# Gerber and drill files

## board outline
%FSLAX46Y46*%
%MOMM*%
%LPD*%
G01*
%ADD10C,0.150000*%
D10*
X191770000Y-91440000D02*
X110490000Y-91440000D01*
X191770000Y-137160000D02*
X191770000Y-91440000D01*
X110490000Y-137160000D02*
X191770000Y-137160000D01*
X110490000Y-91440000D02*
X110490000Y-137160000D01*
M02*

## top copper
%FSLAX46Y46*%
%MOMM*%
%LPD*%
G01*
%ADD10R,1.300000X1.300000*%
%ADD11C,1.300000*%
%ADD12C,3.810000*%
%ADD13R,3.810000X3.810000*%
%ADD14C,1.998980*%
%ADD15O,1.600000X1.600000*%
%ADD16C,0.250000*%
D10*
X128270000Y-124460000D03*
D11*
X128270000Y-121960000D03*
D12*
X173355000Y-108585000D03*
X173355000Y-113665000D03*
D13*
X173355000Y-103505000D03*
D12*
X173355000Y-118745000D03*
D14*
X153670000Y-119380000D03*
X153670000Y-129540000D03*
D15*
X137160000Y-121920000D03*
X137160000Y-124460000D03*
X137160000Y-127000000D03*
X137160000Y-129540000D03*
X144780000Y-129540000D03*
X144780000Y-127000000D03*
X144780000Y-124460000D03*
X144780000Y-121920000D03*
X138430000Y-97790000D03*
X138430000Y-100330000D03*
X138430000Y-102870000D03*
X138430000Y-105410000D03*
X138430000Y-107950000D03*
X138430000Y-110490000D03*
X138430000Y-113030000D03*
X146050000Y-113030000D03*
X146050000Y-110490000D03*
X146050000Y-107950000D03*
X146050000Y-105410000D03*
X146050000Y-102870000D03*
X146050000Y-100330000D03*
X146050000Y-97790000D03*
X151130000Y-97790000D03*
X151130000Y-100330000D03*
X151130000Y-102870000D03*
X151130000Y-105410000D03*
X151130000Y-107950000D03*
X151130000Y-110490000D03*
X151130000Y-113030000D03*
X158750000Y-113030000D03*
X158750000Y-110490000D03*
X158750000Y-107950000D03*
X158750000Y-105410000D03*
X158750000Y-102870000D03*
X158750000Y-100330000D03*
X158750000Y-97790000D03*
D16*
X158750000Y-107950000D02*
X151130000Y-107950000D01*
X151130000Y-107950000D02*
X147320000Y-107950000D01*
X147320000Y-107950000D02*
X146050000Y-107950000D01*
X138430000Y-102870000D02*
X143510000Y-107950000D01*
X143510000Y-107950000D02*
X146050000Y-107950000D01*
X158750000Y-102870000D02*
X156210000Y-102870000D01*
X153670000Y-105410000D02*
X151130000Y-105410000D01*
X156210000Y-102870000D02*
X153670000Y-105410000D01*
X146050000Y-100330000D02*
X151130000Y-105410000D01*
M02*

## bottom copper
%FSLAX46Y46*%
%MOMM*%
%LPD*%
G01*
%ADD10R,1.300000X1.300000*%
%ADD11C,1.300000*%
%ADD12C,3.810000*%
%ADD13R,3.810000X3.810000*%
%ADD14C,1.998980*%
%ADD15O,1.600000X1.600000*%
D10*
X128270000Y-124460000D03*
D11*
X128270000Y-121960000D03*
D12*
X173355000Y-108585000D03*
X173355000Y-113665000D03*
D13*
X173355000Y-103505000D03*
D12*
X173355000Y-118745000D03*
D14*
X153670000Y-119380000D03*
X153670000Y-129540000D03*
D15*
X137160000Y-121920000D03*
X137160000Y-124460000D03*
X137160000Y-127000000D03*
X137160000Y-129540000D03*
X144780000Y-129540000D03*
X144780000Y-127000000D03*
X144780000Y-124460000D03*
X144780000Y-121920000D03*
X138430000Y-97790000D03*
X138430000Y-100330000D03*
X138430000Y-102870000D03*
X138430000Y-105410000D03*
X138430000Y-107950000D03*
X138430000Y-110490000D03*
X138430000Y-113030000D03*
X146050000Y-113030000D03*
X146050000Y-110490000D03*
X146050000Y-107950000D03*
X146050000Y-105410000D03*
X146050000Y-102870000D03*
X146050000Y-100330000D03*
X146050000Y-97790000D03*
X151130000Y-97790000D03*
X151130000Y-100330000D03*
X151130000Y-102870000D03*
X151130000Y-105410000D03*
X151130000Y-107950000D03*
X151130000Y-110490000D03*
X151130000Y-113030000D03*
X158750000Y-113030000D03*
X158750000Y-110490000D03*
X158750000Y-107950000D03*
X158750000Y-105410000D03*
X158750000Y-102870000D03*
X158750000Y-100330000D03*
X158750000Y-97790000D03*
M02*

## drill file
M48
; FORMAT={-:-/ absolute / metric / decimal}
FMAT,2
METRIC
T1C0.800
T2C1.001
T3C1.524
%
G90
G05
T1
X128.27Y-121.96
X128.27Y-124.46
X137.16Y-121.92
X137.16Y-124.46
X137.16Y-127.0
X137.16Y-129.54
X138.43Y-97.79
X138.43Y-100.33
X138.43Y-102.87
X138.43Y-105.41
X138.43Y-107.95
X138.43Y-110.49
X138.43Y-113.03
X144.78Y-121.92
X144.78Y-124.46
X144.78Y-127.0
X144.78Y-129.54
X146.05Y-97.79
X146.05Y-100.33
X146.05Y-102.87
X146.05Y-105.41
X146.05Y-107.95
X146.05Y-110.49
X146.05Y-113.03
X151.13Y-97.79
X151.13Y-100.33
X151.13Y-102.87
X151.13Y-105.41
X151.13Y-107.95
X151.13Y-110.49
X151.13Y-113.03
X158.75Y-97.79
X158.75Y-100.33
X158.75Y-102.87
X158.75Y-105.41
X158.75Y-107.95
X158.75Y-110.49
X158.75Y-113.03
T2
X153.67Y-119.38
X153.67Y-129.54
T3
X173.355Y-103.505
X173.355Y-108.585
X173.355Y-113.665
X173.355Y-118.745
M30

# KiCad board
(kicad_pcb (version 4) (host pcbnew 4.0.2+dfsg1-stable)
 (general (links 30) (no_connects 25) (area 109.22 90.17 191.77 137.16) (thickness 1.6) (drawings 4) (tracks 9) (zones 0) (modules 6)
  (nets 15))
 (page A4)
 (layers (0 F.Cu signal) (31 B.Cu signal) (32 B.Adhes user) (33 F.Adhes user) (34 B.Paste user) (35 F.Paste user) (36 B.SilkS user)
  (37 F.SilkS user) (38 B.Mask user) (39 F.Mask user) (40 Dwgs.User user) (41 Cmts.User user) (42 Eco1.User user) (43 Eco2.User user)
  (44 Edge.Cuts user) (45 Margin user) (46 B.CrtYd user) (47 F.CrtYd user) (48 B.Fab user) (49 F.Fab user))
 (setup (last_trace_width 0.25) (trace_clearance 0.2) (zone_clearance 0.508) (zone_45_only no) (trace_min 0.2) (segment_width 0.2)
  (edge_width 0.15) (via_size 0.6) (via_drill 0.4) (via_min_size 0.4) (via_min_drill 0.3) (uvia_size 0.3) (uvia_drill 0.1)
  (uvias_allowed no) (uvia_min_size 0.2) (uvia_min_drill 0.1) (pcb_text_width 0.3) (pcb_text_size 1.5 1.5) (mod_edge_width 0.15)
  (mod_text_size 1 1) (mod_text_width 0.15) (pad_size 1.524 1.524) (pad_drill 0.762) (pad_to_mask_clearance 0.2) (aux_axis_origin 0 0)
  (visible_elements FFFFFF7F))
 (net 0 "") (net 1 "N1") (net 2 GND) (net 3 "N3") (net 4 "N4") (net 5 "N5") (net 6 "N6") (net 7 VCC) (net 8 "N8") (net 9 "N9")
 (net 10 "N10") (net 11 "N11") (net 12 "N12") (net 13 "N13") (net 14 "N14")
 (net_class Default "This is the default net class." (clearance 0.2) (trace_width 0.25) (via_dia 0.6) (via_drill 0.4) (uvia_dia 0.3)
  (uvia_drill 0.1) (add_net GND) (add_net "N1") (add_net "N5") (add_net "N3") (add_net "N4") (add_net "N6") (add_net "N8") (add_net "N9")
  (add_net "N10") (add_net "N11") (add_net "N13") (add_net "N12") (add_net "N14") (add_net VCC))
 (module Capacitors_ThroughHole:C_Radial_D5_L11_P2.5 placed (layer F.Cu) (at 128.27 124.46 90)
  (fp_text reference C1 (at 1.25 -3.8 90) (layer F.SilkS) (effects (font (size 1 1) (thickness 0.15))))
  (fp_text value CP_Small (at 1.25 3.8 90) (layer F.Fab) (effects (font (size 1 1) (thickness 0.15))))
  (pad 1 thru_hole rect (at 0 0 90) (size 1.3 1.3) (drill 0.8) (layers *.Cu *.Mask F.SilkS) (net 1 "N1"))
  (pad 2 thru_hole circle (at 2.5 0 90) (size 1.3 1.3) (drill 0.8) (layers *.Cu *.Mask F.SilkS) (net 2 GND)))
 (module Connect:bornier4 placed (layer F.Cu) (at 173.355 111.125 270)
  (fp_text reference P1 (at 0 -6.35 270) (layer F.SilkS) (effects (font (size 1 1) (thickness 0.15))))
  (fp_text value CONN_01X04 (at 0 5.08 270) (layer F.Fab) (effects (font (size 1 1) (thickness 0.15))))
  (pad 2 thru_hole circle (at -2.54 0 270) (size 3.81 3.81) (drill 1.524) (layers *.Cu *.Mask F.SilkS) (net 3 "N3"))
  (pad 3 thru_hole circle (at 2.54 0 270) (size 3.81 3.81) (drill 1.524) (layers *.Cu *.Mask F.SilkS) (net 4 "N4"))
  (pad 1 thru_hole rect (at -7.62 0 270) (size 3.81 3.81) (drill 1.524) (layers *.Cu *.Mask F.SilkS) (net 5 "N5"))
  (pad 4 thru_hole circle (at 7.62 0 270) (size 3.81 3.81) (drill 1.524) (layers *.Cu *.Mask F.SilkS) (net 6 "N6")))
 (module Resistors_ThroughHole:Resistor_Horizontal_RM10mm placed (layer F.Cu) (at 153.67 119.38 270)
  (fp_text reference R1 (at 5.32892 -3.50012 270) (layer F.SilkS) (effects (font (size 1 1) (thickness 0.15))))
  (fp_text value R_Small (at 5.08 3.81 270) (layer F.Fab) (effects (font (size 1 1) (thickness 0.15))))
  (pad 1 thru_hole circle (at 0 0 270) (size 1.99898 1.99898) (drill 1.00076) (layers *.Cu *.SilkS *.Mask) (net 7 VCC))
  (pad 2 thru_hole circle (at 10.16 0 270) (size 1.99898 1.99898) (drill 1.00076) (layers *.Cu *.SilkS *.Mask) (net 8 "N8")))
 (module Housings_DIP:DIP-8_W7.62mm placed (layer F.Cu) (at 137.16 121.92)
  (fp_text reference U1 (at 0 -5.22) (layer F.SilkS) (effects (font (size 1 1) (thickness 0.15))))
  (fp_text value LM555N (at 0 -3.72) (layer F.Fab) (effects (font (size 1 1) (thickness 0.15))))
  (pad 1 thru_hole oval (at 0 0) (size 1.6 1.6) (drill 0.8) (layers *.Cu *.Mask F.SilkS) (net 2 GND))
  (pad 2 thru_hole oval (at 0 2.54) (size 1.6 1.6) (drill 0.8) (layers *.Cu *.Mask F.SilkS) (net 1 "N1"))
  (pad 3 thru_hole oval (at 0 5.08) (size 1.6 1.6) (drill 0.8) (layers *.Cu *.Mask F.SilkS) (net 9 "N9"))
  (pad 4 thru_hole oval (at 0 7.62) (size 1.6 1.6) (drill 0.8) (layers *.Cu *.Mask F.SilkS) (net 7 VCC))
  (pad 5 thru_hole oval (at 7.62 7.62) (size 1.6 1.6) (drill 0.8) (layers *.Cu *.Mask F.SilkS) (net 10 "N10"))
  (pad 6 thru_hole oval (at 7.62 5.08) (size 1.6 1.6) (drill 0.8) (layers *.Cu *.Mask F.SilkS) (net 1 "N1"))
  (pad 7 thru_hole oval (at 7.62 2.54) (size 1.6 1.6) (drill 0.8) (layers *.Cu *.Mask F.SilkS) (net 8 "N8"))
  (pad 8 thru_hole oval (at 7.62 0) (size 1.6 1.6) (drill 0.8) (layers *.Cu *.Mask F.SilkS) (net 7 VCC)))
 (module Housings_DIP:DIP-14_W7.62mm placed (layer F.Cu) (at 138.43 97.79)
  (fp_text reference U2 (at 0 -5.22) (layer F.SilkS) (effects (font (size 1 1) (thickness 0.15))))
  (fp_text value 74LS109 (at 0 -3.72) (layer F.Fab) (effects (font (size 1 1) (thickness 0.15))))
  (pad 1 thru_hole oval (at 0 0) (size 1.6 1.6) (drill 0.8) (layers *.Cu *.Mask F.SilkS) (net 7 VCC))
  (pad 2 thru_hole oval (at 0 2.54) (size 1.6 1.6) (drill 0.8) (layers *.Cu *.Mask F.SilkS) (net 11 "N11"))
  (pad 3 thru_hole oval (at 0 5.08) (size 1.6 1.6) (drill 0.8) (layers *.Cu *.Mask F.SilkS) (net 11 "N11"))
  (pad 4 thru_hole oval (at 0 7.62) (size 1.6 1.6) (drill 0.8) (layers *.Cu *.Mask F.SilkS) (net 9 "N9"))
  (pad 5 thru_hole oval (at 0 10.16) (size 1.6 1.6) (drill 0.8) (layers *.Cu *.Mask F.SilkS) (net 7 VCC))
  (pad 6 thru_hole oval (at 0 12.7) (size 1.6 1.6) (drill 0.8) (layers *.Cu *.Mask F.SilkS) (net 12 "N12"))
  (pad 7 thru_hole oval (at 0 15.24) (size 1.6 1.6) (drill 0.8) (layers *.Cu *.Mask F.SilkS) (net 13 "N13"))
  (pad 8 thru_hole oval (at 7.62 15.24) (size 1.6 1.6) (drill 0.8) (layers *.Cu *.Mask F.SilkS) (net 2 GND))
  (pad 9 thru_hole oval (at 7.62 12.7) (size 1.6 1.6) (drill 0.8) (layers *.Cu *.Mask F.SilkS) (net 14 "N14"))
  (pad 10 thru_hole oval (at 7.62 10.16) (size 1.6 1.6) (drill 0.8) (layers *.Cu *.Mask F.SilkS) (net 11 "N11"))
  (pad 11 thru_hole oval (at 7.62 7.62) (size 1.6 1.6) (drill 0.8) (layers *.Cu *.Mask F.SilkS) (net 7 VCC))
  (pad 12 thru_hole oval (at 7.62 5.08) (size 1.6 1.6) (drill 0.8) (layers *.Cu *.Mask F.SilkS) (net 9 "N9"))
  (pad 13 thru_hole oval (at 7.62 2.54) (size 1.6 1.6) (drill 0.8) (layers *.Cu *.Mask F.SilkS) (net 13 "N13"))
  (pad 14 thru_hole oval (at 7.62 0) (size 1.6 1.6) (drill 0.8) (layers *.Cu *.Mask F.SilkS) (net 13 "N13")))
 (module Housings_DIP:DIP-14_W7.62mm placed (layer F.Cu) (at 151.13 97.79)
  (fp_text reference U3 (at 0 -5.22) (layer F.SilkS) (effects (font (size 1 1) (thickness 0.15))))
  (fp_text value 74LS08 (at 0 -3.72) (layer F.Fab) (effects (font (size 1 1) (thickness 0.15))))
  (pad 1 thru_hole oval (at 0 0) (size 1.6 1.6) (drill 0.8) (layers *.Cu *.Mask F.SilkS) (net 12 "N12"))
  (pad 2 thru_hole oval (at 0 2.54) (size 1.6 1.6) (drill 0.8) (layers *.Cu *.Mask F.SilkS) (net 14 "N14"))
  (pad 3 thru_hole oval (at 0 5.08) (size 1.6 1.6) (drill 0.8) (layers *.Cu *.Mask F.SilkS) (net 5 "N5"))
  (pad 4 thru_hole oval (at 0 7.62) (size 1.6 1.6) (drill 0.8) (layers *.Cu *.Mask F.SilkS) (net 13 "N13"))
  (pad 5 thru_hole oval (at 0 10.16) (size 1.6 1.6) (drill 0.8) (layers *.Cu *.Mask F.SilkS) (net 11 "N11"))
  (pad 6 thru_hole oval (at 0 12.7) (size 1.6 1.6) (drill 0.8) (layers *.Cu *.Mask F.SilkS) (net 3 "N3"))
  (pad 7 thru_hole oval (at 0 15.24) (size 1.6 1.6) (drill 0.8) (layers *.Cu *.Mask F.SilkS) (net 2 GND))
  (pad 8 thru_hole oval (at 7.62 15.24) (size 1.6 1.6) (drill 0.8) (layers *.Cu *.Mask F.SilkS) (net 4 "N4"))
  (pad 9 thru_hole oval (at 7.62 12.7) (size 1.6 1.6) (drill 0.8) (layers *.Cu *.Mask F.SilkS) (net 13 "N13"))
  (pad 10 thru_hole oval (at 7.62 10.16) (size 1.6 1.6) (drill 0.8) (layers *.Cu *.Mask F.SilkS) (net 11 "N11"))
  (pad 11 thru_hole oval (at 7.62 7.62) (size 1.6 1.6) (drill 0.8) (layers *.Cu *.Mask F.SilkS) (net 6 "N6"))
  (pad 12 thru_hole oval (at 7.62 5.08) (size 1.6 1.6) (drill 0.8) (layers *.Cu *.Mask F.SilkS) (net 13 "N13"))
  (pad 13 thru_hole oval (at 7.62 2.54) (size 1.6 1.6) (drill 0.8) (layers *.Cu *.Mask F.SilkS) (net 14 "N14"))
  (pad 14 thru_hole oval (at 7.62 0) (size 1.6 1.6) (drill 0.8) (layers *.Cu *.Mask F.SilkS) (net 7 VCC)))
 (gr_line (start 191.77 91.44) (end 110.49 91.44) (angle 90) (layer Edge.Cuts) (width 0.15))
 (gr_line (start 191.77 137.16) (end 191.77 91.44) (angle 90) (layer Edge.Cuts) (width 0.15))
 (gr_line (start 110.49 137.16) (end 191.77 137.16) (angle 90) (layer Edge.Cuts) (width 0.15))
 (gr_line (start 110.49 91.44) (end 110.49 137.16) (angle 90) (layer Edge.Cuts) (width 0.15))
 (segment (start 158.75 107.95) (end 151.13 107.95) (width 0.25) (layer F.Cu) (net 11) (status C00000))
 (segment (start 151.13 107.95) (end 147.32 107.95) (width 0.25) (layer F.Cu) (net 11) (status 400000))
 (segment (start 147.32 107.95) (end 146.05 107.95) (width 0.25) (layer F.Cu) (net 11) (status 800000))
 (segment (start 138.43 102.87) (end 143.51 107.95) (width 0.25) (layer F.Cu) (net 11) (status 400000))
 (segment (start 143.51 107.95) (end 146.05 107.95) (width 0.25) (layer F.Cu) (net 11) (status 800000))
 (segment (start 158.75 102.87) (end 156.21 102.87) (width 0.25) (layer F.Cu) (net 13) (status 400000))
 (segment (start 153.67 105.41) (end 151.13 105.41) (width 0.25) (layer F.Cu) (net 13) (status 800000))
 (segment (start 156.21 102.87) (end 153.67 105.41) (width 0.25) (layer F.Cu) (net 13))
 (segment (start 146.05 100.33) (end 151.13 105.41) (width 0.25) (layer F.Cu) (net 13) (status C00000)))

